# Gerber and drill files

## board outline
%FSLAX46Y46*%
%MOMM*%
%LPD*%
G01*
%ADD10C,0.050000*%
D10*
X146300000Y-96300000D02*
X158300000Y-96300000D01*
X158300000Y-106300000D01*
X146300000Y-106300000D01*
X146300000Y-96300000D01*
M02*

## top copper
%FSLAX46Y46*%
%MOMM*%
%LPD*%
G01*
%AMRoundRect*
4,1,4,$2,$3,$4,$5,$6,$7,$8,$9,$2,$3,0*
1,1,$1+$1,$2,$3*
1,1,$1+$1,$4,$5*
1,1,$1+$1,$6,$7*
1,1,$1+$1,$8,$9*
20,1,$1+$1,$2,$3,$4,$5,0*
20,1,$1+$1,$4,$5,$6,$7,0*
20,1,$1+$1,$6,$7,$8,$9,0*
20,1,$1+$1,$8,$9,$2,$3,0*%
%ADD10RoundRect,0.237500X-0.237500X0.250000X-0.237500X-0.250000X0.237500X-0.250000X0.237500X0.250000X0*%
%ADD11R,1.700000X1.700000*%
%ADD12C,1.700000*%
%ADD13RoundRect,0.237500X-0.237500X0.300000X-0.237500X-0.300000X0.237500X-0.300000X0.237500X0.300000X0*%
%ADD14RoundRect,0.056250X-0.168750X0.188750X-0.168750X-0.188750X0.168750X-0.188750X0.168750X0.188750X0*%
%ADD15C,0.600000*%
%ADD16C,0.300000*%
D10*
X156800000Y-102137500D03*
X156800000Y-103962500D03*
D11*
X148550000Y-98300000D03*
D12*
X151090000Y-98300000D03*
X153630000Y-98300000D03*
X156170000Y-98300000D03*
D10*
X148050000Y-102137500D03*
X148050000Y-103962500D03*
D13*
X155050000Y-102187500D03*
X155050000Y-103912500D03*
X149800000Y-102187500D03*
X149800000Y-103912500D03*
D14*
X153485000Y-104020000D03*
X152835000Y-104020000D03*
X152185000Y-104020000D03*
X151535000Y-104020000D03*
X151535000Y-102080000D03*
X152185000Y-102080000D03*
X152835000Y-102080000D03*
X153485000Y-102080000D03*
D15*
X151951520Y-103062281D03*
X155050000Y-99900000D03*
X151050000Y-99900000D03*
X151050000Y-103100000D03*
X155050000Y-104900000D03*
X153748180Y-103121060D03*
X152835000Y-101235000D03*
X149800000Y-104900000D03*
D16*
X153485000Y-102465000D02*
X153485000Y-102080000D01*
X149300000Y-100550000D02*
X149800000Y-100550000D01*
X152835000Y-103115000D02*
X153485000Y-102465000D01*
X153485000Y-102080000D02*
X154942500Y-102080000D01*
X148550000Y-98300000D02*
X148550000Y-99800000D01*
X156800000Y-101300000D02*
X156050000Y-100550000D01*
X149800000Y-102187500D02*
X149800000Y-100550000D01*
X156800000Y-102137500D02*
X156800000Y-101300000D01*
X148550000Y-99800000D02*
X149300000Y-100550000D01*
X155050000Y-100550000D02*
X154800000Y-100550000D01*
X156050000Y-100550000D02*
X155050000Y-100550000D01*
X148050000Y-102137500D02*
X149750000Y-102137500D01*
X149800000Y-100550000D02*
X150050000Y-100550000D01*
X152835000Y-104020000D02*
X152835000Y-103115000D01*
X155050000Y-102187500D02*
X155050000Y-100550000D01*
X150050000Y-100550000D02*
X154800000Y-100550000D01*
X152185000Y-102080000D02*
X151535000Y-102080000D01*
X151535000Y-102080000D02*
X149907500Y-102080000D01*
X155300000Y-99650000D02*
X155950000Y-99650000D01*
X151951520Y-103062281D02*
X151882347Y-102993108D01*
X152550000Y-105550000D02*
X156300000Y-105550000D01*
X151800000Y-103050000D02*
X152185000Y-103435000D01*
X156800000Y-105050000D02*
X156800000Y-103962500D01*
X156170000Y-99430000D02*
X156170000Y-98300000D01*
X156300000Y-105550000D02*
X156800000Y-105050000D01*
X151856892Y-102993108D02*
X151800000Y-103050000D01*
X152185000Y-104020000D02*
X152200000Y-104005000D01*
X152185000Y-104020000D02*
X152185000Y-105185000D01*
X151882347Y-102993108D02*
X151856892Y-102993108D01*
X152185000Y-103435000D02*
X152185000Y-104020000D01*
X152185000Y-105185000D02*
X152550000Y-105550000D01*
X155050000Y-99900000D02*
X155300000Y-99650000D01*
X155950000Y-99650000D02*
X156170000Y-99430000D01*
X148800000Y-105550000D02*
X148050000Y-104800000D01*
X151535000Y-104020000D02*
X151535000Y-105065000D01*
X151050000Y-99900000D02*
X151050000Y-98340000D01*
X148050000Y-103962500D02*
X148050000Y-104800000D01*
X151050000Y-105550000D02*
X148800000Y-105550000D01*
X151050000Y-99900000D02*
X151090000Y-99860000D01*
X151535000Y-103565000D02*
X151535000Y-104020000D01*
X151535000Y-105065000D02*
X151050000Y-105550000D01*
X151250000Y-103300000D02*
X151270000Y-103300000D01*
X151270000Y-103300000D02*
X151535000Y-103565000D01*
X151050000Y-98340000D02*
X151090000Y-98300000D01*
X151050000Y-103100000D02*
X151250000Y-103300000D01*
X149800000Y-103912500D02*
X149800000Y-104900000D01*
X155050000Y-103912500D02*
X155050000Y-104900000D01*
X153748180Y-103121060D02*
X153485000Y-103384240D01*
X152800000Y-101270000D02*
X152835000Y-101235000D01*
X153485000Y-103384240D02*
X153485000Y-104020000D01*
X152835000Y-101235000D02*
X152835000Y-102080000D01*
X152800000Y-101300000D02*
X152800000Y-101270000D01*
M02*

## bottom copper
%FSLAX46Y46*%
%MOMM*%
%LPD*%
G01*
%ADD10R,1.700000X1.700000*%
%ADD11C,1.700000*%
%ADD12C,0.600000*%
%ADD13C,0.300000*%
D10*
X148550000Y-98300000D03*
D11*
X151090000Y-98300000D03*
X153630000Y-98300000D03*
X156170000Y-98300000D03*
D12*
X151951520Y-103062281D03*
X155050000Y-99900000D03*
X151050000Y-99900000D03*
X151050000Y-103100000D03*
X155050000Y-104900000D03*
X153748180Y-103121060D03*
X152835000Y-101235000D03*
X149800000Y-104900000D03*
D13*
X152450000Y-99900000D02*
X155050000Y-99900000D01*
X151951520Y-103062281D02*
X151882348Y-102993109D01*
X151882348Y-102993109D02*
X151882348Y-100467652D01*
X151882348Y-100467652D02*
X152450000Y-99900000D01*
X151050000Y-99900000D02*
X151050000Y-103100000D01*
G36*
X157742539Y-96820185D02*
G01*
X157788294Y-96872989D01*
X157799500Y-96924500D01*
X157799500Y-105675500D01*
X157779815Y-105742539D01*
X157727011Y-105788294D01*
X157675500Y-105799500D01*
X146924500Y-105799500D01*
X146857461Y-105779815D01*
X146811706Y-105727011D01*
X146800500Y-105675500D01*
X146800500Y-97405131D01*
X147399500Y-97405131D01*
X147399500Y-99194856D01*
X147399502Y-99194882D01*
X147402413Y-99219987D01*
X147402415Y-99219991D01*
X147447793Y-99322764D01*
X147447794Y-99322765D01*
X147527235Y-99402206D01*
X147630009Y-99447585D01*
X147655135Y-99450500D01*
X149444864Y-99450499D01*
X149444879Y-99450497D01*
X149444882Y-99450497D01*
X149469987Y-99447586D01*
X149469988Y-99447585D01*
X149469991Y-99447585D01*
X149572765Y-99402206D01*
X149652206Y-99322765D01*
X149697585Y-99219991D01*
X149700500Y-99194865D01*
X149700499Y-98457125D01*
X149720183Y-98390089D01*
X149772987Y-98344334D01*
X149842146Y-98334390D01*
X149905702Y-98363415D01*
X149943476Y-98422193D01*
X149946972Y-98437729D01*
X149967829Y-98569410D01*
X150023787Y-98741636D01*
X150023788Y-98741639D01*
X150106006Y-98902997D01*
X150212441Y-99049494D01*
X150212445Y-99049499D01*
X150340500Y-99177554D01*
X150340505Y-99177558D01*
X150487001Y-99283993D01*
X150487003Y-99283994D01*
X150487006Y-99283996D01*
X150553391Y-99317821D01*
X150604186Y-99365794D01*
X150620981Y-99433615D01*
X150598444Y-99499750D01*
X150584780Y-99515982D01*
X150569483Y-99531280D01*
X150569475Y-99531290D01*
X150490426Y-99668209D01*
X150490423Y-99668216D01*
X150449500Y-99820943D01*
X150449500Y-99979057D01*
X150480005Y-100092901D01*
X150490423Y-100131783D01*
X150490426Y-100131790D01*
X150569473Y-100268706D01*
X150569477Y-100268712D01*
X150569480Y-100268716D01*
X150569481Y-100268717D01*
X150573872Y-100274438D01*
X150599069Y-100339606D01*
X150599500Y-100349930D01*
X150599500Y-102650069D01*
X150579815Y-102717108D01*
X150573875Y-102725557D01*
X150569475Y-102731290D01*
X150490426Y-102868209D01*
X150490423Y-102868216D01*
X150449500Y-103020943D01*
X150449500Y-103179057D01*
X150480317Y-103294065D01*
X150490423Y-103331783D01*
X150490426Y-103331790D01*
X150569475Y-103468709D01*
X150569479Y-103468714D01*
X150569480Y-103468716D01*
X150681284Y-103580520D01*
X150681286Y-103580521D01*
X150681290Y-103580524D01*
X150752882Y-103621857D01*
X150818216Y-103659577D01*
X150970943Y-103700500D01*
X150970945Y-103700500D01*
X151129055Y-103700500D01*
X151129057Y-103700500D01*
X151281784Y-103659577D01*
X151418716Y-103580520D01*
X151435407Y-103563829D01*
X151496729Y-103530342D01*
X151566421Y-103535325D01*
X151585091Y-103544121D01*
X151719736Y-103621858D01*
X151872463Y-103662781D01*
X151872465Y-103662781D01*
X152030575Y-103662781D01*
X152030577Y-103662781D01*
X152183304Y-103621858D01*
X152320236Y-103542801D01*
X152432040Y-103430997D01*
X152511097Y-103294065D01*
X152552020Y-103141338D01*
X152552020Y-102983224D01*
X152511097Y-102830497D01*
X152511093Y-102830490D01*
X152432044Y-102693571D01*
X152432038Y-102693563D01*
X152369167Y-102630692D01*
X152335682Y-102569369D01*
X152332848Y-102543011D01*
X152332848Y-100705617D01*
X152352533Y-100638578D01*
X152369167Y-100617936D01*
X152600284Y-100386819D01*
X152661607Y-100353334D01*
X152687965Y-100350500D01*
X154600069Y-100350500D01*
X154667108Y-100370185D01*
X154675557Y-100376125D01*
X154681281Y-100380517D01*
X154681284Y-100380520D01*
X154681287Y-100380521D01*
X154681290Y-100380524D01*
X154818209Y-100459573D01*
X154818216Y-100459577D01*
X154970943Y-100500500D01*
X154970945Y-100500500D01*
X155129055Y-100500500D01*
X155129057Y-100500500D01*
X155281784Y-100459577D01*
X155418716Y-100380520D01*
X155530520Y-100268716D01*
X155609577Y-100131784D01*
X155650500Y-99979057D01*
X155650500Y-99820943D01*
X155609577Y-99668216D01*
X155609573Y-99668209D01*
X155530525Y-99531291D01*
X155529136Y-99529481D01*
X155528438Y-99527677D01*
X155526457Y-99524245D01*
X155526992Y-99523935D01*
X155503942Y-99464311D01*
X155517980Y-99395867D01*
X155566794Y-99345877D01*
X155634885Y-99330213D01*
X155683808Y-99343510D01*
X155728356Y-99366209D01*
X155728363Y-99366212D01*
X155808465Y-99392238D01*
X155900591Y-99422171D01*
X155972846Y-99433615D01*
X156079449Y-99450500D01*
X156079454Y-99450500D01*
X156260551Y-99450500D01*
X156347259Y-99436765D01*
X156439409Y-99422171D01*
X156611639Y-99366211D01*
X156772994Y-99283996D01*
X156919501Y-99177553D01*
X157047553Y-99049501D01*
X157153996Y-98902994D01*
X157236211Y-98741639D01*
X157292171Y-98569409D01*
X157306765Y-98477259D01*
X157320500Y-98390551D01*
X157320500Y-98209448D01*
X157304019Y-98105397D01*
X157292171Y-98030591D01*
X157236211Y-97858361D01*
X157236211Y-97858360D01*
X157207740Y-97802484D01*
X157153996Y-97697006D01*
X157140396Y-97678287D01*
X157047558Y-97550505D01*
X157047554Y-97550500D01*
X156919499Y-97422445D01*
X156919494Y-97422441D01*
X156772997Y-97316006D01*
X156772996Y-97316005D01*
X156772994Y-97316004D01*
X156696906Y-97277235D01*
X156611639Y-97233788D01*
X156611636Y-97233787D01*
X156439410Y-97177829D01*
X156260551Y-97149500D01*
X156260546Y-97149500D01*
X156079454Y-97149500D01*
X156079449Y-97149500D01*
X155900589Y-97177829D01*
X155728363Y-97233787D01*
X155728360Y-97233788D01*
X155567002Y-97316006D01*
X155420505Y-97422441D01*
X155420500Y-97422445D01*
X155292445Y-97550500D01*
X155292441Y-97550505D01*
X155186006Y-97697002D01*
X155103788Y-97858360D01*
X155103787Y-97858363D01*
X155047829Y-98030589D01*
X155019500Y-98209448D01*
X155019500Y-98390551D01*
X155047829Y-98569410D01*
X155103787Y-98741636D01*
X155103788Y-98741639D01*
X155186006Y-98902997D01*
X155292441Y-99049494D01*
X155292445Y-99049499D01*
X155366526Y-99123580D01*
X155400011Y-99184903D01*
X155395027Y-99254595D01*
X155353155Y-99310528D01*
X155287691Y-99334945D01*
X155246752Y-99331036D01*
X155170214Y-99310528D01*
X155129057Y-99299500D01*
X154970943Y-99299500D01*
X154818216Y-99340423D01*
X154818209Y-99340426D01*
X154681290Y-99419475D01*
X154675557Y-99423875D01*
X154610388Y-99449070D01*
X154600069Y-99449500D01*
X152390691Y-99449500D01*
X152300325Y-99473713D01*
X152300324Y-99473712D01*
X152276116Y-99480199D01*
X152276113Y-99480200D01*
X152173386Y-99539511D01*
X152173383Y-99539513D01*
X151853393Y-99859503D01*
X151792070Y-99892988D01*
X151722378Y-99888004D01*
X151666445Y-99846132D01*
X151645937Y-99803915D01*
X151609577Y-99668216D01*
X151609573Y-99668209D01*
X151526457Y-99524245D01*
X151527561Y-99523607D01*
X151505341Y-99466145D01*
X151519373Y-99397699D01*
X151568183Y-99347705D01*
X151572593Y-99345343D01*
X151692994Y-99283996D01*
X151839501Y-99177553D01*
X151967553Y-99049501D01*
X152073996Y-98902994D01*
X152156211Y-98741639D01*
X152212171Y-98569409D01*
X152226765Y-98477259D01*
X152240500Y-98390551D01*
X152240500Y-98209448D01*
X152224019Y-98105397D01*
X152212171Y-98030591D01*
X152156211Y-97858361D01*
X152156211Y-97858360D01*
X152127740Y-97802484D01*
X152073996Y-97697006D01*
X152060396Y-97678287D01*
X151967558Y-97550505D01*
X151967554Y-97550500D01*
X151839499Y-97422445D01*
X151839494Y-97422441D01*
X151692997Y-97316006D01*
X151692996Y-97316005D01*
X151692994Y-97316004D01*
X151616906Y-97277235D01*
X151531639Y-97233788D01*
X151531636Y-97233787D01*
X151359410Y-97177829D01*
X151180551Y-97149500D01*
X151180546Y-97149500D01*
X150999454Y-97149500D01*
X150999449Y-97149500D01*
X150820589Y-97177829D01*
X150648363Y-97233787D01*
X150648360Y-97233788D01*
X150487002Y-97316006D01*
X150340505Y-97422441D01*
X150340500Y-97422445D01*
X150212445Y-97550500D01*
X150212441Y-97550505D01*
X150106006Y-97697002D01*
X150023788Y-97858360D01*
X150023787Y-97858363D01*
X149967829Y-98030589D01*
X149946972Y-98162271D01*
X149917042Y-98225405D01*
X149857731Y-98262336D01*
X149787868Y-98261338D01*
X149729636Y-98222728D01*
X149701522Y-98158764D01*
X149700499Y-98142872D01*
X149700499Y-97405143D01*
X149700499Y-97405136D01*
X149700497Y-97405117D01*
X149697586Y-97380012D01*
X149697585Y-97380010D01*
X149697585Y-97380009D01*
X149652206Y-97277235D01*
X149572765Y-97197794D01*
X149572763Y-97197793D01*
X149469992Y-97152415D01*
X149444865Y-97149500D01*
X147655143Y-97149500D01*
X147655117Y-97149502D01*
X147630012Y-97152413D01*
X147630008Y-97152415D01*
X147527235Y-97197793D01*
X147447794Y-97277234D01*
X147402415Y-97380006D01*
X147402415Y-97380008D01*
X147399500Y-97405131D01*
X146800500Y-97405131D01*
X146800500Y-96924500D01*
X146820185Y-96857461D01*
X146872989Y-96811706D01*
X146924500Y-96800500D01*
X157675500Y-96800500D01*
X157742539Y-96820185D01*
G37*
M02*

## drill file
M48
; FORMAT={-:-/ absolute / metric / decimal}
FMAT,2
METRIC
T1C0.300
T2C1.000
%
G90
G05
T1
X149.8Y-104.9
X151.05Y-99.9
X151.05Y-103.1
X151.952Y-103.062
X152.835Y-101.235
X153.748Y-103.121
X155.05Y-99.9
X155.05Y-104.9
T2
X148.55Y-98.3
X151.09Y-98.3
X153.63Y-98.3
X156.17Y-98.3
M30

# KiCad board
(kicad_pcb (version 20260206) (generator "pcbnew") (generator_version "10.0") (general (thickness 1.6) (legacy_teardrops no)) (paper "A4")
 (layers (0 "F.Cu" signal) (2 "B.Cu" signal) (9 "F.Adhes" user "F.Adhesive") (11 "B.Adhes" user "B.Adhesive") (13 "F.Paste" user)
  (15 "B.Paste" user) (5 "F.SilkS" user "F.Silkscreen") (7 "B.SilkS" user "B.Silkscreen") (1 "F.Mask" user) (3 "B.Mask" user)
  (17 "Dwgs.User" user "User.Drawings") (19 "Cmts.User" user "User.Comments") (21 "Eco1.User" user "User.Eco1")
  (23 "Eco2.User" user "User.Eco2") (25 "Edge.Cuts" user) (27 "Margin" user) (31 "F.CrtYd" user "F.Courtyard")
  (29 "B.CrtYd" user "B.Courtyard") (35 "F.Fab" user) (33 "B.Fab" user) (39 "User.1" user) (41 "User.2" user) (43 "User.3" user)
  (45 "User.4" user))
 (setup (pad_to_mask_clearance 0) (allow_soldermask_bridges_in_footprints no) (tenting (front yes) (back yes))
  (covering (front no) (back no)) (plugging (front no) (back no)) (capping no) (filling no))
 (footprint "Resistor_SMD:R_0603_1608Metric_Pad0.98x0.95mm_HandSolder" (layer "F.Cu") (at 156.8 103.05 -90)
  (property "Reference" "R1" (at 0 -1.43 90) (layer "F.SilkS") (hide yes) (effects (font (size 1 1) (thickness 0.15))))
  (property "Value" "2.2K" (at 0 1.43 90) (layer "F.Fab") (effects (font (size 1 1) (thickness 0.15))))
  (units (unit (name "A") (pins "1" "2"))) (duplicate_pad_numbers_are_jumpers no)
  (pad "1" smd roundrect (at -0.9125 0 270) (size 0.975 0.95) (layers "F.Cu" "F.Mask" "F.Paste") (roundrect_rratio 0.25) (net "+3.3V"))
  (pad "2" smd roundrect (at 0.9125 0 270) (size 0.975 0.95) (layers "F.Cu" "F.Mask" "F.Paste") (roundrect_rratio 0.25) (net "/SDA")))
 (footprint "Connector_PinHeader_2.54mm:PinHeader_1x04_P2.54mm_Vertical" (layer "F.Cu") (at 148.55 98.3 90)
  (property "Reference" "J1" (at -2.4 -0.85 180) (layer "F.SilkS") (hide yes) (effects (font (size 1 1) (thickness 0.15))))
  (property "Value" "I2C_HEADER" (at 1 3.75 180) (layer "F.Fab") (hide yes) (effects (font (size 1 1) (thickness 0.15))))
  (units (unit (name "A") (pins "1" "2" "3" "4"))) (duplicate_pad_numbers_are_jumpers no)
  (pad "1" thru_hole rect (at 0 0 90) (size 1.7 1.7) (drill 1) (layers "*.Cu" "*.Mask") (remove_unused_layers no) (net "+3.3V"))
  (pad "2" thru_hole circle (at 0 2.54 90) (size 1.7 1.7) (drill 1) (layers "*.Cu" "*.Mask") (remove_unused_layers no) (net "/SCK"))
  (pad "3" thru_hole circle (at 0 5.08 90) (size 1.7 1.7) (drill 1) (layers "*.Cu" "*.Mask") (remove_unused_layers no) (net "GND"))
  (pad "4" thru_hole circle (at 0 7.62 90) (size 1.7 1.7) (drill 1) (layers "*.Cu" "*.Mask") (remove_unused_layers no) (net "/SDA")))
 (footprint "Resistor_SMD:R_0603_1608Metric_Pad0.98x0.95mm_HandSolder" (layer "F.Cu") (at 148.05 103.05 -90)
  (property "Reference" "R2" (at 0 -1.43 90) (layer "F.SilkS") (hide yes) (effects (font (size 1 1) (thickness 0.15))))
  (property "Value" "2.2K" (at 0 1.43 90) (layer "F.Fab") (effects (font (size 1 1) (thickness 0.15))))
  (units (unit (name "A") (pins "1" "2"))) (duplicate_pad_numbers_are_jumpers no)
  (pad "1" smd roundrect (at -0.9125 0 270) (size 0.975 0.95) (layers "F.Cu" "F.Mask" "F.Paste") (roundrect_rratio 0.25) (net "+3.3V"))
  (pad "2" smd roundrect (at 0.9125 0 270) (size 0.975 0.95) (layers "F.Cu" "F.Mask" "F.Paste") (roundrect_rratio 0.25) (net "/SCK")))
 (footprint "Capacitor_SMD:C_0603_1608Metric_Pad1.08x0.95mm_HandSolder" (layer "F.Cu") (at 155.05 103.05 -90)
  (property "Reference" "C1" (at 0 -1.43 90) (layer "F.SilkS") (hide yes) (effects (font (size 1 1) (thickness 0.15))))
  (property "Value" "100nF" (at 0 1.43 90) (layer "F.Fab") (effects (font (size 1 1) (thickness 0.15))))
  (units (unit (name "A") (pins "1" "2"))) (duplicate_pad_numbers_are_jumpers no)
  (pad "1" smd roundrect (at -0.8625 0 270) (size 1.075 0.95) (layers "F.Cu" "F.Mask" "F.Paste") (roundrect_rratio 0.25) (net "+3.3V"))
  (pad "2" smd roundrect (at 0.8625 0 270) (size 1.075 0.95) (layers "F.Cu" "F.Mask" "F.Paste") (roundrect_rratio 0.25) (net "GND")))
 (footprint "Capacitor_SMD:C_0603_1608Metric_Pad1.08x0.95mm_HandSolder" (layer "F.Cu") (at 149.8 103.05 -90)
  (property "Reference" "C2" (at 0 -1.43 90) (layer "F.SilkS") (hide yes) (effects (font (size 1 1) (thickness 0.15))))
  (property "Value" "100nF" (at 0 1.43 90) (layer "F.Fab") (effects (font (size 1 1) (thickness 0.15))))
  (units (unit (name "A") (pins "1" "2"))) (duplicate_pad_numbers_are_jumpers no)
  (pad "1" smd roundrect (at -0.8625 0 270) (size 1.075 0.95) (layers "F.Cu" "F.Mask" "F.Paste") (roundrect_rratio 0.25) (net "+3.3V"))
  (pad "2" smd roundrect (at 0.8625 0 270) (size 1.075 0.95) (layers "F.Cu" "F.Mask" "F.Paste") (roundrect_rratio 0.25) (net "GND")))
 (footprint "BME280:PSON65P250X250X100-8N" (layer "F.Cu") (at 152.51 103.05 -90)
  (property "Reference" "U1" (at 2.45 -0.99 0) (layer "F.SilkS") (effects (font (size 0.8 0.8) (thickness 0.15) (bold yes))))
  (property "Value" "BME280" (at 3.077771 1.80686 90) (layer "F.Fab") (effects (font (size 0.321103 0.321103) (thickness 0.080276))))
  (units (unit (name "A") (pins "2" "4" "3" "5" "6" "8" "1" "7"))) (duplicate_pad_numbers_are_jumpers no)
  (pad "1" smd roundrect (at 0.97 -0.975 270) (size 0.49 0.45) (layers "F.Cu" "F.Mask" "F.Paste") (roundrect_rratio 0.125) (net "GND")
   (solder_mask_margin 0.102))
  (pad "2" smd roundrect (at 0.97 -0.325 270) (size 0.49 0.45) (layers "F.Cu" "F.Mask" "F.Paste") (roundrect_rratio 0.125) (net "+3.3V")
   (solder_mask_margin 0.102))
  (pad "3" smd roundrect (at 0.97 0.325 270) (size 0.49 0.45) (layers "F.Cu" "F.Mask" "F.Paste") (roundrect_rratio 0.125) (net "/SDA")
   (solder_mask_margin 0.102))
  (pad "4" smd roundrect (at 0.97 0.975 270) (size 0.49 0.45) (layers "F.Cu" "F.Mask" "F.Paste") (roundrect_rratio 0.125) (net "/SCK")
   (solder_mask_margin 0.102))
  (pad "5" smd roundrect (at -0.97 0.975 270) (size 0.49 0.45) (layers "F.Cu" "F.Mask" "F.Paste") (roundrect_rratio 0.125) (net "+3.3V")
   (solder_mask_margin 0.102))
  (pad "6" smd roundrect (at -0.97 0.325 270) (size 0.49 0.45) (layers "F.Cu" "F.Mask" "F.Paste") (roundrect_rratio 0.125) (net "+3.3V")
   (solder_mask_margin 0.102))
  (pad "7" smd roundrect (at -0.97 -0.325 270) (size 0.49 0.45) (layers "F.Cu" "F.Mask" "F.Paste") (roundrect_rratio 0.125) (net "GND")
   (solder_mask_margin 0.102))
  (pad "8" smd roundrect (at -0.97 -0.975 270) (size 0.49 0.45) (layers "F.Cu" "F.Mask" "F.Paste") (roundrect_rratio 0.125) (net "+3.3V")
   (solder_mask_margin 0.102)))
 (gr_rect (start 146.3 96.3) (end 158.3 106.3) (stroke (width 0.05) (type default)) (fill no) (layer "Edge.Cuts"))
 (segment (start 153.485 102.465) (end 153.485 102.08) (width 0.3) (layer "F.Cu") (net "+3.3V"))
 (segment (start 149.3 100.55) (end 149.8 100.55) (width 0.3) (layer "F.Cu") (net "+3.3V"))
 (segment (start 152.835 103.115) (end 153.485 102.465) (width 0.3) (layer "F.Cu") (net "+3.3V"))
 (segment (start 153.485 102.08) (end 154.9425 102.08) (width 0.3) (layer "F.Cu") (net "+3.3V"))
 (segment (start 148.55 98.3) (end 148.55 99.8) (width 0.3) (layer "F.Cu") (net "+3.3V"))
 (segment (start 156.8 101.3) (end 156.05 100.55) (width 0.3) (layer "F.Cu") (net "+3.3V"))
 (segment (start 149.8 102.1875) (end 149.8 100.55) (width 0.3) (layer "F.Cu") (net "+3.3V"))
 (segment (start 156.8 102.1375) (end 156.8 101.3) (width 0.3) (layer "F.Cu") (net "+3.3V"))
 (segment (start 148.55 99.8) (end 149.3 100.55) (width 0.3) (layer "F.Cu") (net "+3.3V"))
 (segment (start 155.05 100.55) (end 154.8 100.55) (width 0.3) (layer "F.Cu") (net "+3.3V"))
 (segment (start 156.05 100.55) (end 155.05 100.55) (width 0.3) (layer "F.Cu") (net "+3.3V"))
 (segment (start 148.05 102.1375) (end 149.75 102.1375) (width 0.3) (layer "F.Cu") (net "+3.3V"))
 (segment (start 149.8 100.55) (end 150.05 100.55) (width 0.3) (layer "F.Cu") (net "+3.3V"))
 (segment (start 152.835 104.02) (end 152.835 103.115) (width 0.3) (layer "F.Cu") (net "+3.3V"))
 (segment (start 155.05 102.1875) (end 155.05 100.55) (width 0.3) (layer "F.Cu") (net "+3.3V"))
 (segment (start 150.05 100.55) (end 154.8 100.55) (width 0.3) (layer "F.Cu") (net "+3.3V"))
 (segment (start 152.185 102.08) (end 151.535 102.08) (width 0.3) (layer "F.Cu") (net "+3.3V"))
 (segment (start 151.535 102.08) (end 149.9075 102.08) (width 0.3) (layer "F.Cu") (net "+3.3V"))
 (segment (start 155.3 99.65) (end 155.95 99.65) (width 0.3) (layer "F.Cu") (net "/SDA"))
 (segment (start 151.95152 103.062281) (end 151.882347 102.993108) (width 0.3) (layer "F.Cu") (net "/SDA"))
 (segment (start 152.55 105.55) (end 156.3 105.55) (width 0.3) (layer "F.Cu") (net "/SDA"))
 (segment (start 151.8 103.05) (end 152.185 103.435) (width 0.3) (layer "F.Cu") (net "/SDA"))
 (segment (start 156.8 105.05) (end 156.8 103.9625) (width 0.3) (layer "F.Cu") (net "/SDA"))
 (segment (start 156.17 99.43) (end 156.17 98.3) (width 0.3) (layer "F.Cu") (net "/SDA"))
 (segment (start 156.3 105.55) (end 156.8 105.05) (width 0.3) (layer "F.Cu") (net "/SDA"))
 (segment (start 151.856892 102.993108) (end 151.8 103.05) (width 0.3) (layer "F.Cu") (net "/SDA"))
 (segment (start 152.185 104.02) (end 152.2 104.005) (width 0.3) (layer "F.Cu") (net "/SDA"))
 (segment (start 152.185 104.02) (end 152.185 105.185) (width 0.3) (layer "F.Cu") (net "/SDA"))
 (segment (start 151.882347 102.993108) (end 151.856892 102.993108) (width 0.3) (layer "F.Cu") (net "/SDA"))
 (segment (start 152.185 103.435) (end 152.185 104.02) (width 0.3) (layer "F.Cu") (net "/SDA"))
 (segment (start 152.185 105.185) (end 152.55 105.55) (width 0.3) (layer "F.Cu") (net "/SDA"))
 (segment (start 155.05 99.9) (end 155.3 99.65) (width 0.3) (layer "F.Cu") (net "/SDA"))
 (segment (start 155.95 99.65) (end 156.17 99.43) (width 0.3) (layer "F.Cu") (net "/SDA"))
 (via (at 151.95152 103.062281) (size 0.6) (drill 0.3) (layers "F.Cu" "B.Cu") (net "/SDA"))
 (via (at 155.05 99.9) (size 0.6) (drill 0.3) (layers "F.Cu" "B.Cu") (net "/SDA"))
 (segment (start 152.45 99.9) (end 155.05 99.9) (width 0.3) (layer "B.Cu") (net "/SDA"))
 (segment (start 151.95152 103.062281) (end 151.882348 102.993109) (width 0.3) (layer "B.Cu") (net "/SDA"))
 (segment (start 151.882348 102.993109) (end 151.882348 100.467652) (width 0.3) (layer "B.Cu") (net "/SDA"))
 (segment (start 151.882348 100.467652) (end 152.45 99.9) (width 0.3) (layer "B.Cu") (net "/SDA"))
 (segment (start 148.8 105.55) (end 148.05 104.8) (width 0.3) (layer "F.Cu") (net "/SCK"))
 (segment (start 151.535 104.02) (end 151.535 105.065) (width 0.3) (layer "F.Cu") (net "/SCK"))
 (segment (start 151.05 99.9) (end 151.05 98.34) (width 0.3) (layer "F.Cu") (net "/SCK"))
 (segment (start 148.05 103.9625) (end 148.05 104.8) (width 0.3) (layer "F.Cu") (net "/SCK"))
 (segment (start 151.05 105.55) (end 148.8 105.55) (width 0.3) (layer "F.Cu") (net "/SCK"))
 (segment (start 151.05 99.9) (end 151.09 99.86) (width 0.3) (layer "F.Cu") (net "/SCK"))
 (segment (start 151.535 103.565) (end 151.535 104.02) (width 0.3) (layer "F.Cu") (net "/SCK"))
 (segment (start 151.535 105.065) (end 151.05 105.55) (width 0.3) (layer "F.Cu") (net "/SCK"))
 (segment (start 151.25 103.3) (end 151.27 103.3) (width 0.3) (layer "F.Cu") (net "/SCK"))
 (segment (start 151.27 103.3) (end 151.535 103.565) (width 0.3) (layer "F.Cu") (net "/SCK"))
 (segment (start 151.05 98.34) (end 151.09 98.3) (width 0.3) (layer "F.Cu") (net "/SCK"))
 (segment (start 151.05 103.1) (end 151.25 103.3) (width 0.3) (layer "F.Cu") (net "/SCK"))
 (via (at 151.05 99.9) (size 0.6) (drill 0.3) (layers "F.Cu" "B.Cu") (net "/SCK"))
 (via (at 151.05 103.1) (size 0.6) (drill 0.3) (layers "F.Cu" "B.Cu") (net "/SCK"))
 (segment (start 151.05 99.9) (end 151.05 103.1) (width 0.3) (layer "B.Cu") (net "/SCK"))
 (segment (start 149.8 103.9125) (end 149.8 104.9) (width 0.3) (layer "F.Cu") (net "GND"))
 (segment (start 155.05 103.9125) (end 155.05 104.9) (width 0.3) (layer "F.Cu") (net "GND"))
 (segment (start 153.74818 103.12106) (end 153.485 103.38424) (width 0.3) (layer "F.Cu") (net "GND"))
 (segment (start 152.8 101.27) (end 152.835 101.235) (width 0.3) (layer "F.Cu") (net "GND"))
 (segment (start 153.485 103.38424) (end 153.485 104.02) (width 0.3) (layer "F.Cu") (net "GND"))
 (segment (start 152.835 101.235) (end 152.835 102.08) (width 0.3) (layer "F.Cu") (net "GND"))
 (segment (start 152.8 101.3) (end 152.8 101.27) (width 0.3) (layer "F.Cu") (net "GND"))
 (via (at 155.05 104.9) (size 0.6) (drill 0.3) (layers "F.Cu" "B.Cu") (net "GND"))
 (via (at 153.74818 103.12106) (size 0.6) (drill 0.3) (layers "F.Cu" "B.Cu") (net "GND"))
 (via (at 152.835 101.235) (size 0.6) (drill 0.3) (layers "F.Cu" "B.Cu") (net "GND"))
 (via (at 149.8 104.9) (size 0.6) (drill 0.3) (layers "F.Cu" "B.Cu") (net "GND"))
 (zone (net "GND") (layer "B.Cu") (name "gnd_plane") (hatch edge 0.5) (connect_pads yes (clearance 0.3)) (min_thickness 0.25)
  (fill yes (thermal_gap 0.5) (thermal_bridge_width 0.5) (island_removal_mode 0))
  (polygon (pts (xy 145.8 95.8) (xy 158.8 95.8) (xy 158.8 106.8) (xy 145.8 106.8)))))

